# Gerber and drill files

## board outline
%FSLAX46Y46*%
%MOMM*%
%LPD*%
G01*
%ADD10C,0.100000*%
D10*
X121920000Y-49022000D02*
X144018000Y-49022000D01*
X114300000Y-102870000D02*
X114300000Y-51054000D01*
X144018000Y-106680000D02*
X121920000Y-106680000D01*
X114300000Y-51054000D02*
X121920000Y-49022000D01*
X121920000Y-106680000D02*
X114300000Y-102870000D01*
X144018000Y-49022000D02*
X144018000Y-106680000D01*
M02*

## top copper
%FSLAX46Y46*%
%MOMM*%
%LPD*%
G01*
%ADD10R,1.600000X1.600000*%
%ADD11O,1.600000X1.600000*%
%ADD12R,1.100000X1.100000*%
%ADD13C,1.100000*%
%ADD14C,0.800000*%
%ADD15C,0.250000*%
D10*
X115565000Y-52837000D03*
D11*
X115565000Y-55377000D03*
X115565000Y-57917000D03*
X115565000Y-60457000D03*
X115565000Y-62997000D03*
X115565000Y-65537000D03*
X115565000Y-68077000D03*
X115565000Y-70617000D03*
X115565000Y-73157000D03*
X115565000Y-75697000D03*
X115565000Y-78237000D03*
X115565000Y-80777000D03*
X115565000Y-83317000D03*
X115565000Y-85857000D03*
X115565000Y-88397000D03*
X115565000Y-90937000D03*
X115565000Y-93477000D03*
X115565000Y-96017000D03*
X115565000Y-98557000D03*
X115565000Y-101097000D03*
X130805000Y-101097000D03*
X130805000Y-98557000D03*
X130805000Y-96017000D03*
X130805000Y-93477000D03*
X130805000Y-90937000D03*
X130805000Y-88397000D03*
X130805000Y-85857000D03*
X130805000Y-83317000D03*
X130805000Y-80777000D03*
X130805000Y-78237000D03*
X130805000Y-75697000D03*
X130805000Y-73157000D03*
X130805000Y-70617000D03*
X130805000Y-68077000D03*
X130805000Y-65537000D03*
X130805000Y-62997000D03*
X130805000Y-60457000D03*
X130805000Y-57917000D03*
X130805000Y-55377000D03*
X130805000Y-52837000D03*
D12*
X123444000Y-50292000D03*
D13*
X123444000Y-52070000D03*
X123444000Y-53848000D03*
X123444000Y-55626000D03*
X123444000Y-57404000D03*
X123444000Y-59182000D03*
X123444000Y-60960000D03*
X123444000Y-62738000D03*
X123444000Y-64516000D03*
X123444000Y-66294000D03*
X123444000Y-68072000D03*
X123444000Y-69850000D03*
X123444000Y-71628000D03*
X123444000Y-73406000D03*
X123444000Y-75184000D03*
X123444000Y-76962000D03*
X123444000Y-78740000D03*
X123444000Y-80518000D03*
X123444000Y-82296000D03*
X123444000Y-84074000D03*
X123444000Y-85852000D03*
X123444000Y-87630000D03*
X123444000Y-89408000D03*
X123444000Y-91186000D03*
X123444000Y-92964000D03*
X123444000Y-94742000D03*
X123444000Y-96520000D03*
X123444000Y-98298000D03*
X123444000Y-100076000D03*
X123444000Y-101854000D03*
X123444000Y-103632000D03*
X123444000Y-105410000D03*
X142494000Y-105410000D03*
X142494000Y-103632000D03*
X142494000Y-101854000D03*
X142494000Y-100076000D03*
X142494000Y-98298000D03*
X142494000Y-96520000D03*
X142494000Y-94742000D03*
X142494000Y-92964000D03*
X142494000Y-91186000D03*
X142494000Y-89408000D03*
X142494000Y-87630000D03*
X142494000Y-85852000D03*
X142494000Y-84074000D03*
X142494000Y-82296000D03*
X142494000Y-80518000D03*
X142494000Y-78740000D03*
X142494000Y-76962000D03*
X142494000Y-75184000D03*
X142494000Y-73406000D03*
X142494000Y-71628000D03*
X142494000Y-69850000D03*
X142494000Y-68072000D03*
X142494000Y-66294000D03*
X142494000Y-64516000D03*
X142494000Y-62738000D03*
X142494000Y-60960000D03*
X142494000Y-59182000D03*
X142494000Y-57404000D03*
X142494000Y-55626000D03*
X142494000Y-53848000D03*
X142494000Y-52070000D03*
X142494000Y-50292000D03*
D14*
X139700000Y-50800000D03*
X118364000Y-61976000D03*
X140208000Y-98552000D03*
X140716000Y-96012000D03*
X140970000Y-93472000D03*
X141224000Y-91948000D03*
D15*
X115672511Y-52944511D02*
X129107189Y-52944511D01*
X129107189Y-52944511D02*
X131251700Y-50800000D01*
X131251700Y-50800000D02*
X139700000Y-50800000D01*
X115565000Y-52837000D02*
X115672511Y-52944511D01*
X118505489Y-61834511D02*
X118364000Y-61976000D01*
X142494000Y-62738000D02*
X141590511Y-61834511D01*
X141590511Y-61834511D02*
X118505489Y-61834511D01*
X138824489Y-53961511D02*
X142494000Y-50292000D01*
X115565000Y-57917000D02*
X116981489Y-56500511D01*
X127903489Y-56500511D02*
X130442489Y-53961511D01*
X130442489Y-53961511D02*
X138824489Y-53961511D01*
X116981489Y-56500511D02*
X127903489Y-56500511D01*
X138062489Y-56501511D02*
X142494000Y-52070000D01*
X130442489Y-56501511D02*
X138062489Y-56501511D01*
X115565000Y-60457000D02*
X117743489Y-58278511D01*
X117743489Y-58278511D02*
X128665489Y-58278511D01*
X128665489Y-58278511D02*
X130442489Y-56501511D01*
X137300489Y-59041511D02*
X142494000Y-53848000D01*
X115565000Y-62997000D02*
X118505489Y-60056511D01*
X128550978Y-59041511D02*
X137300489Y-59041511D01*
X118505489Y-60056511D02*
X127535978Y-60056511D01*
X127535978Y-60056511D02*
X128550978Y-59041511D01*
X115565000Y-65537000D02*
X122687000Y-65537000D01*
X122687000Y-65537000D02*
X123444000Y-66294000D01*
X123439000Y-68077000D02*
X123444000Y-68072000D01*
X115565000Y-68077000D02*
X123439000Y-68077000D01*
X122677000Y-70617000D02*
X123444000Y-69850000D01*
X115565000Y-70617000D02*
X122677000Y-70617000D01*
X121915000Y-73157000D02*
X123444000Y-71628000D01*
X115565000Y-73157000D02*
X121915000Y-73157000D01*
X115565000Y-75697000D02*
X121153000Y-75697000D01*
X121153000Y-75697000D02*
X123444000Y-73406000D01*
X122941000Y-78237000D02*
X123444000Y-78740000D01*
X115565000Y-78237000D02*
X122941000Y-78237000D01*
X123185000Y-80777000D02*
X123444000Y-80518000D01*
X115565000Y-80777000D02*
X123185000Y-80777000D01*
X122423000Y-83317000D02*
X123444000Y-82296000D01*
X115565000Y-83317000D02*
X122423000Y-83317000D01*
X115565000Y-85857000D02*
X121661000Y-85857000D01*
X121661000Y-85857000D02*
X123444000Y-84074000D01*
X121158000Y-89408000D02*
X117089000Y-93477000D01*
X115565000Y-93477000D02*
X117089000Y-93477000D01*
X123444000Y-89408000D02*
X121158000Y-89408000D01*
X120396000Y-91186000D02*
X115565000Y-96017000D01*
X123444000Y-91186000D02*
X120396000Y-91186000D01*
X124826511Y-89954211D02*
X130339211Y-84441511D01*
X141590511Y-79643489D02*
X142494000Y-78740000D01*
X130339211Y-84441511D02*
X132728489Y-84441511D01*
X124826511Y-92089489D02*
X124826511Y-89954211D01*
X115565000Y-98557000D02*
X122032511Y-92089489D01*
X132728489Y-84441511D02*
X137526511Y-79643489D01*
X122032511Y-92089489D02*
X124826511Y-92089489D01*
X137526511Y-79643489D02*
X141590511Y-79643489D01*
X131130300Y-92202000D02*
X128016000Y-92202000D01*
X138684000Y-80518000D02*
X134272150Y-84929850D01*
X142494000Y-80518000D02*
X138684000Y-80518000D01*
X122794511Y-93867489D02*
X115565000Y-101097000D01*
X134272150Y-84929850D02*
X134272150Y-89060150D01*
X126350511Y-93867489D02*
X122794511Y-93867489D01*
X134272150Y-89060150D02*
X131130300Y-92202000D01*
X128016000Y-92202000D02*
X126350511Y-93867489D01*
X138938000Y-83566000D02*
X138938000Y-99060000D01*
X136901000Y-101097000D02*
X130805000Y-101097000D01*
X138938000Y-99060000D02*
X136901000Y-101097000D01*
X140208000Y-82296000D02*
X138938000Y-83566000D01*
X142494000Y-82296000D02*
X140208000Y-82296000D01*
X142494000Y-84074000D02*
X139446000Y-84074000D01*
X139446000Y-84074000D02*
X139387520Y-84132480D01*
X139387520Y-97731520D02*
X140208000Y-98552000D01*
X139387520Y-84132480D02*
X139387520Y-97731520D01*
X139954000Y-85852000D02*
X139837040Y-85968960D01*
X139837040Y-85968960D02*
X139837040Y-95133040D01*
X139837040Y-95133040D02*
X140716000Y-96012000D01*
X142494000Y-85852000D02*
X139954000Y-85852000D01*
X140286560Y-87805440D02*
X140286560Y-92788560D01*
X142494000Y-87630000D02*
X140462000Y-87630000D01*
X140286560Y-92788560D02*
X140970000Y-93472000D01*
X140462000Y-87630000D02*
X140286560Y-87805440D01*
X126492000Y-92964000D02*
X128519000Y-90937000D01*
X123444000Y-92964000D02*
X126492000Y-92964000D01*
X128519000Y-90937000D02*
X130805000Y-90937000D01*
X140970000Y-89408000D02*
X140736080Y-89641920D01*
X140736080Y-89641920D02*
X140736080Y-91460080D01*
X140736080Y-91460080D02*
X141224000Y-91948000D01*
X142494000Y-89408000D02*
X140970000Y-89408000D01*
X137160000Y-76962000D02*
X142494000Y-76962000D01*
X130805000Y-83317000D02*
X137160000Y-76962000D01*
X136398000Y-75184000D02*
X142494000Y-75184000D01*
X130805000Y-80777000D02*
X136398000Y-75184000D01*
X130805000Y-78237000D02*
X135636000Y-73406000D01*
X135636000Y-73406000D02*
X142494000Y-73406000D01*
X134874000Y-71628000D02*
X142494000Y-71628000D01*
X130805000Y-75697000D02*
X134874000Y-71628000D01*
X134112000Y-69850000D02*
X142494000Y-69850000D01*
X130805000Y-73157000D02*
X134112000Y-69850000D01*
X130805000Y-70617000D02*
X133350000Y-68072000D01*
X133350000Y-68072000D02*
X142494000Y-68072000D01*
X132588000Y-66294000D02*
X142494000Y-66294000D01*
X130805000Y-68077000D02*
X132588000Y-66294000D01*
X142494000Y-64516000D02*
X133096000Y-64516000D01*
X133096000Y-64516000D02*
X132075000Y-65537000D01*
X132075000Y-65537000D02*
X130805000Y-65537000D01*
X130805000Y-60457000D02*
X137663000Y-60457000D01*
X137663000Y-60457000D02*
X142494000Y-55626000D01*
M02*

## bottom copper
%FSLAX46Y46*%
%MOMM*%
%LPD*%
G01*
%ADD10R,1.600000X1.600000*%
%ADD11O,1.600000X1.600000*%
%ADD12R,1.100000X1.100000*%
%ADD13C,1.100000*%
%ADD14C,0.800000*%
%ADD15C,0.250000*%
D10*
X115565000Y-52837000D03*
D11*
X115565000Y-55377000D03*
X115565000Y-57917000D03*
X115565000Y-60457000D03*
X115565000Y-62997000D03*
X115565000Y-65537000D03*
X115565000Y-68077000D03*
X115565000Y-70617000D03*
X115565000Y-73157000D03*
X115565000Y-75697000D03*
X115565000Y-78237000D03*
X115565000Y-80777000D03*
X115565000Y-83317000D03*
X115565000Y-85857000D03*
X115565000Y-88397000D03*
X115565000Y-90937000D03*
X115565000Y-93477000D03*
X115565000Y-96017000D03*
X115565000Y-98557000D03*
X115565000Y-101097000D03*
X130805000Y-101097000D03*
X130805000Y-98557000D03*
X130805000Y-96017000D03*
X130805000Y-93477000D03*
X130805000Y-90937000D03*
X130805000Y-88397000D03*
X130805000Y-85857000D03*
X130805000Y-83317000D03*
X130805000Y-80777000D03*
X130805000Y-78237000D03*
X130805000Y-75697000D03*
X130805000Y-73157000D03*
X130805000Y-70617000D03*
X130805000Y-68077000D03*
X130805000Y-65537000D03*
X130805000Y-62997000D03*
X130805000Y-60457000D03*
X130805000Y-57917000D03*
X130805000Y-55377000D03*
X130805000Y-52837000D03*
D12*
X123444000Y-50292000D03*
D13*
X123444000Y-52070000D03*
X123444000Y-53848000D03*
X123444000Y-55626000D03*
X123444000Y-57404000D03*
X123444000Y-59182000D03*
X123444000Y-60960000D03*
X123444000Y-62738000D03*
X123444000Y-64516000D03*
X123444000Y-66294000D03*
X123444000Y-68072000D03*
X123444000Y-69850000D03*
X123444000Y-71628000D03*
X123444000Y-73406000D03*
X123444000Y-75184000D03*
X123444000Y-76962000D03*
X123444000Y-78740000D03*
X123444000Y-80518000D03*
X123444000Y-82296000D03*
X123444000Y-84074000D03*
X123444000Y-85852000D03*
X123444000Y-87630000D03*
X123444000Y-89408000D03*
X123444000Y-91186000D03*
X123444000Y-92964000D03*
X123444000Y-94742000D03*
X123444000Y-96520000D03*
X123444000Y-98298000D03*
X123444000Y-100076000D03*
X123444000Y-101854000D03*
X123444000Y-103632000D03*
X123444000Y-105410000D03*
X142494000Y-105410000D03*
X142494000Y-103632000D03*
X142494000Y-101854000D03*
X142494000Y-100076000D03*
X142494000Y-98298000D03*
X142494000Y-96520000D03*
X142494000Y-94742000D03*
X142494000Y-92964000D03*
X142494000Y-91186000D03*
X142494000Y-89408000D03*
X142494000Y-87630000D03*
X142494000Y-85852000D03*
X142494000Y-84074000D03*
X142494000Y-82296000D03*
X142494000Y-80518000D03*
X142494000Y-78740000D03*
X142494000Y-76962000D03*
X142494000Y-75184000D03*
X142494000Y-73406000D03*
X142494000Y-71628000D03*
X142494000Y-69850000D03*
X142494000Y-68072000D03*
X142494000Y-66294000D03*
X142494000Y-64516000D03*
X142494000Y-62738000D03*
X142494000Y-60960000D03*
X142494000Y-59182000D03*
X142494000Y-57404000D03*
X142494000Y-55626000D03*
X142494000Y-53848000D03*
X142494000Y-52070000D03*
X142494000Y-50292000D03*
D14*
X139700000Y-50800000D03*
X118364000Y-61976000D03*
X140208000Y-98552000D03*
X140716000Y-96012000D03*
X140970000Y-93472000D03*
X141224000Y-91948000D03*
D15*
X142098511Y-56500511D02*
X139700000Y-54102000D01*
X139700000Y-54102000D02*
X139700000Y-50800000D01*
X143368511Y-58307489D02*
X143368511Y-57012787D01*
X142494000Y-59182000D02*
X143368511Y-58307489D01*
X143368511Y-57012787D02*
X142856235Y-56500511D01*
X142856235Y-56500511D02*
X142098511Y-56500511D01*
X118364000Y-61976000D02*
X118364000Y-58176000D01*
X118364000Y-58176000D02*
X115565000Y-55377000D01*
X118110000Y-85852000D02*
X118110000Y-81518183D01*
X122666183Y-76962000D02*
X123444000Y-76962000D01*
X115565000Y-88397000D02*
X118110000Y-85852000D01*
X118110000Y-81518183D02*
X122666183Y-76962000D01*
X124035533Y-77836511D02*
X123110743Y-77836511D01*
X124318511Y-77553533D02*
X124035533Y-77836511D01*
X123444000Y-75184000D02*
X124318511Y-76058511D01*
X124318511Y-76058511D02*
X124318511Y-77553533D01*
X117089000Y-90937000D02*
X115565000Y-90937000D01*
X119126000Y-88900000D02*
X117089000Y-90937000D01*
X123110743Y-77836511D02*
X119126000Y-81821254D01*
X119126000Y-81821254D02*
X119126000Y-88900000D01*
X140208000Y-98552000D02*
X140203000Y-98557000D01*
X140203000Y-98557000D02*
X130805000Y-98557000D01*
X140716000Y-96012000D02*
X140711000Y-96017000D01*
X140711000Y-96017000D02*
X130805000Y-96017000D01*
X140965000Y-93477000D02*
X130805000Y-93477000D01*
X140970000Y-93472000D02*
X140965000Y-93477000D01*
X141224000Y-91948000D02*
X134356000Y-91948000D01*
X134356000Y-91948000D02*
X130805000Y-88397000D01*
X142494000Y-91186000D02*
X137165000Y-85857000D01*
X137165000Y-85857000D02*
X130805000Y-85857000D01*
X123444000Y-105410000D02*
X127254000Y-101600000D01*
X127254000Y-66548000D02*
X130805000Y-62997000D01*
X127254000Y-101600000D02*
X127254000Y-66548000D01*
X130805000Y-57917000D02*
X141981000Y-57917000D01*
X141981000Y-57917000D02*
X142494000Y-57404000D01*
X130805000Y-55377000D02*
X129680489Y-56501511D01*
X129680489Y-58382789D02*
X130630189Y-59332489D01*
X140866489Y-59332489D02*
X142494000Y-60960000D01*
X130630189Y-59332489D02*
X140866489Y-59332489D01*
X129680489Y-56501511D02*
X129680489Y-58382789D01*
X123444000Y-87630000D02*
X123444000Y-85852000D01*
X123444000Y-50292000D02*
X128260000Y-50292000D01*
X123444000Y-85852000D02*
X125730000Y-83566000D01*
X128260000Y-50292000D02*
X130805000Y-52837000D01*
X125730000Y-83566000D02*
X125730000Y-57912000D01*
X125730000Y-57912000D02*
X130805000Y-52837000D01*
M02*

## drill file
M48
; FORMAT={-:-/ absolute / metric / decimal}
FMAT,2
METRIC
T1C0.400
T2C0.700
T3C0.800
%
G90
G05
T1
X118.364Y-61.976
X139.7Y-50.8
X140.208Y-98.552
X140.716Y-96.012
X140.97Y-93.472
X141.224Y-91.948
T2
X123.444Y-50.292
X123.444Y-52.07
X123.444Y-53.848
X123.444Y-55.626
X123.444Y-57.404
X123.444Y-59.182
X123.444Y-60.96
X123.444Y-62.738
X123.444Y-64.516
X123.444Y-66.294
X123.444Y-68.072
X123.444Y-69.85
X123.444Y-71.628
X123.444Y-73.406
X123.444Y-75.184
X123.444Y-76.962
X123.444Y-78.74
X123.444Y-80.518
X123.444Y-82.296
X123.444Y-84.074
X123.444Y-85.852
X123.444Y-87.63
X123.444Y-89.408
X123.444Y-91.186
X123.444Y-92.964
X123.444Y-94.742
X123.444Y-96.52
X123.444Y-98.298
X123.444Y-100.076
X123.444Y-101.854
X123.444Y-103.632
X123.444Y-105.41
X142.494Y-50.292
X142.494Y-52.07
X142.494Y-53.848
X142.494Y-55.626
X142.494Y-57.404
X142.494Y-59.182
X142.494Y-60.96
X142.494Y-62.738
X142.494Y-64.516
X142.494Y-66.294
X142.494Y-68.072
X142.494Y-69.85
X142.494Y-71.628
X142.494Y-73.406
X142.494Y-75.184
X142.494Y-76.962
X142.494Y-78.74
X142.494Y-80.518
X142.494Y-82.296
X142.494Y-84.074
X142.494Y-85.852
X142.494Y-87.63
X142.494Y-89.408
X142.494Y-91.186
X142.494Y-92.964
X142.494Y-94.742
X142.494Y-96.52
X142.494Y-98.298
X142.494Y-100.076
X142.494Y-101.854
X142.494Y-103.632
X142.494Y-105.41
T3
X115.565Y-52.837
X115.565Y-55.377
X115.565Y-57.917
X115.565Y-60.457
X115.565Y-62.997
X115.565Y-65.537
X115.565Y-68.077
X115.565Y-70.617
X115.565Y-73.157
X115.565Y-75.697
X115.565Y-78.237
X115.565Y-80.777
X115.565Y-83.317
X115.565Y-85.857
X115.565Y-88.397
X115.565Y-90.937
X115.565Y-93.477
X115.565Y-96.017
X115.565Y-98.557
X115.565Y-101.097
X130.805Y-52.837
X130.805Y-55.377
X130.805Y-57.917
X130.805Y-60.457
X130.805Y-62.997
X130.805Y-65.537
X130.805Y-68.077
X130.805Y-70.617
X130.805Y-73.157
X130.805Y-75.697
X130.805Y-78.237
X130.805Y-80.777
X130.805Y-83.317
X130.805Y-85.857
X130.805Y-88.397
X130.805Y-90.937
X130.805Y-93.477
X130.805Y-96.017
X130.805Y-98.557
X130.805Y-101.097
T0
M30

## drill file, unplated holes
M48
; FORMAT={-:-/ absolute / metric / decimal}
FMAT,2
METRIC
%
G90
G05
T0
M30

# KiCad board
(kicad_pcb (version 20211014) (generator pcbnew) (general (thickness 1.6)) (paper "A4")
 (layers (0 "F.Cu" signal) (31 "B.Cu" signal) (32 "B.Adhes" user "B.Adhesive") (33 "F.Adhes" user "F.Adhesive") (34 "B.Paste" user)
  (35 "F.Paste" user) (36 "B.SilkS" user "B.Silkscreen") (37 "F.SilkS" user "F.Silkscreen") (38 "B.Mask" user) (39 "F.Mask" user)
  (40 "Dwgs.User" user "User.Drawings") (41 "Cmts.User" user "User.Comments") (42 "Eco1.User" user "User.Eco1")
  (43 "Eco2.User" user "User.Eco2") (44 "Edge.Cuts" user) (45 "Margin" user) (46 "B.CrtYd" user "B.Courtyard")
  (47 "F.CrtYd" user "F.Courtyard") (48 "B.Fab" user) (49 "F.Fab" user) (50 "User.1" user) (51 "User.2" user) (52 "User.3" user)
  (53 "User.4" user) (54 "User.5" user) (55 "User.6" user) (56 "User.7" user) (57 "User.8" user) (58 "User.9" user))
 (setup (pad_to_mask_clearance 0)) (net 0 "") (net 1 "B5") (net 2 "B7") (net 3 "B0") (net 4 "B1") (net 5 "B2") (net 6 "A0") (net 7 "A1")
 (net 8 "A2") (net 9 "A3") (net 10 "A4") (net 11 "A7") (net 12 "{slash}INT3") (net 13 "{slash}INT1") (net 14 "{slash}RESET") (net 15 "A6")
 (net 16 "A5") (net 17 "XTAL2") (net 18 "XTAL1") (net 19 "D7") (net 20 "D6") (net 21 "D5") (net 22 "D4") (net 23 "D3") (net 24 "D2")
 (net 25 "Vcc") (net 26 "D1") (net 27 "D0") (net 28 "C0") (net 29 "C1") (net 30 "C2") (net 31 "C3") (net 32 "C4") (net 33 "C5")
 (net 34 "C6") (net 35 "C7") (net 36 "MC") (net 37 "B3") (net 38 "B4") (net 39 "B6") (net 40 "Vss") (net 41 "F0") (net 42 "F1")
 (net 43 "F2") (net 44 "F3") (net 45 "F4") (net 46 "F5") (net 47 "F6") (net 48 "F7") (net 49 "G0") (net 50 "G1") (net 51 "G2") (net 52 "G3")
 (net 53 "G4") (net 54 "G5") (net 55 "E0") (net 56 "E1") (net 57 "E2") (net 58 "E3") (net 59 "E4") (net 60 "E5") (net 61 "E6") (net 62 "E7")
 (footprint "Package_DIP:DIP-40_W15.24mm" (layer "F.Cu") (at 115.565 52.837)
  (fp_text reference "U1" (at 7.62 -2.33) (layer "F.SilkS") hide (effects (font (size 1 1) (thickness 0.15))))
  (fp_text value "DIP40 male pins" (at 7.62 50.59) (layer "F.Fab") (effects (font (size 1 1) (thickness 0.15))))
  (pad "1" thru_hole rect locked (at 0 0) (size 1.6 1.6) (drill 0.8) (layers *.Cu *.Mask) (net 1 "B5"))
  (pad "2" thru_hole oval locked (at 0 2.54) (size 1.6 1.6) (drill 0.8) (layers *.Cu *.Mask) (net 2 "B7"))
  (pad "3" thru_hole oval locked (at 0 5.08) (size 1.6 1.6) (drill 0.8) (layers *.Cu *.Mask) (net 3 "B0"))
  (pad "4" thru_hole oval locked (at 0 7.62) (size 1.6 1.6) (drill 0.8) (layers *.Cu *.Mask) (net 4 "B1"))
  (pad "5" thru_hole oval locked (at 0 10.16) (size 1.6 1.6) (drill 0.8) (layers *.Cu *.Mask) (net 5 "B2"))
  (pad "6" thru_hole oval locked (at 0 12.7) (size 1.6 1.6) (drill 0.8) (layers *.Cu *.Mask) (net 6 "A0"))
  (pad "7" thru_hole oval locked (at 0 15.24) (size 1.6 1.6) (drill 0.8) (layers *.Cu *.Mask) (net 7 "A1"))
  (pad "8" thru_hole oval locked (at 0 17.78) (size 1.6 1.6) (drill 0.8) (layers *.Cu *.Mask) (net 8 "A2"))
  (pad "9" thru_hole oval locked (at 0 20.32) (size 1.6 1.6) (drill 0.8) (layers *.Cu *.Mask) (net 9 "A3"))
  (pad "10" thru_hole oval locked (at 0 22.86) (size 1.6 1.6) (drill 0.8) (layers *.Cu *.Mask) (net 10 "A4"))
  (pad "11" thru_hole oval locked (at 0 25.4) (size 1.6 1.6) (drill 0.8) (layers *.Cu *.Mask) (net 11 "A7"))
  (pad "12" thru_hole oval locked (at 0 27.94) (size 1.6 1.6) (drill 0.8) (layers *.Cu *.Mask) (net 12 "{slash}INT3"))
  (pad "13" thru_hole oval locked (at 0 30.48) (size 1.6 1.6) (drill 0.8) (layers *.Cu *.Mask) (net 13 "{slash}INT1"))
  (pad "14" thru_hole oval locked (at 0 33.02) (size 1.6 1.6) (drill 0.8) (layers *.Cu *.Mask) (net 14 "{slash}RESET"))
  (pad "15" thru_hole oval locked (at 0 35.56) (size 1.6 1.6) (drill 0.8) (layers *.Cu *.Mask) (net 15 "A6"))
  (pad "16" thru_hole oval locked (at 0 38.1) (size 1.6 1.6) (drill 0.8) (layers *.Cu *.Mask) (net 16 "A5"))
  (pad "17" thru_hole oval locked (at 0 40.64) (size 1.6 1.6) (drill 0.8) (layers *.Cu *.Mask) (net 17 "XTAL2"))
  (pad "18" thru_hole oval locked (at 0 43.18) (size 1.6 1.6) (drill 0.8) (layers *.Cu *.Mask) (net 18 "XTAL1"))
  (pad "19" thru_hole oval locked (at 0 45.72) (size 1.6 1.6) (drill 0.8) (layers *.Cu *.Mask) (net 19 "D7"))
  (pad "20" thru_hole oval locked (at 0 48.26) (size 1.6 1.6) (drill 0.8) (layers *.Cu *.Mask) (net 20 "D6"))
  (pad "21" thru_hole oval locked (at 15.24 48.26) (size 1.6 1.6) (drill 0.8) (layers *.Cu *.Mask) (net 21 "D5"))
  (pad "22" thru_hole oval locked (at 15.24 45.72) (size 1.6 1.6) (drill 0.8) (layers *.Cu *.Mask) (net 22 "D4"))
  (pad "23" thru_hole oval locked (at 15.24 43.18) (size 1.6 1.6) (drill 0.8) (layers *.Cu *.Mask) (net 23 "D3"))
  (pad "24" thru_hole oval locked (at 15.24 40.64) (size 1.6 1.6) (drill 0.8) (layers *.Cu *.Mask) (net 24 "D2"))
  (pad "25" thru_hole oval locked (at 15.24 38.1) (size 1.6 1.6) (drill 0.8) (layers *.Cu *.Mask) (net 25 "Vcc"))
  (pad "26" thru_hole oval locked (at 15.24 35.56) (size 1.6 1.6) (drill 0.8) (layers *.Cu *.Mask) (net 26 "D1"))
  (pad "27" thru_hole oval locked (at 15.24 33.02) (size 1.6 1.6) (drill 0.8) (layers *.Cu *.Mask) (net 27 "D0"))
  (pad "28" thru_hole oval locked (at 15.24 30.48) (size 1.6 1.6) (drill 0.8) (layers *.Cu *.Mask) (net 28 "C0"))
  (pad "29" thru_hole oval locked (at 15.24 27.94) (size 1.6 1.6) (drill 0.8) (layers *.Cu *.Mask) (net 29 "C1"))
  (pad "30" thru_hole oval locked (at 15.24 25.4) (size 1.6 1.6) (drill 0.8) (layers *.Cu *.Mask) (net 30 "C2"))
  (pad "31" thru_hole oval locked (at 15.24 22.86) (size 1.6 1.6) (drill 0.8) (layers *.Cu *.Mask) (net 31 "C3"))
  (pad "32" thru_hole oval locked (at 15.24 20.32) (size 1.6 1.6) (drill 0.8) (layers *.Cu *.Mask) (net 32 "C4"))
  (pad "33" thru_hole oval locked (at 15.24 17.78) (size 1.6 1.6) (drill 0.8) (layers *.Cu *.Mask) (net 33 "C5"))
  (pad "34" thru_hole oval locked (at 15.24 15.24) (size 1.6 1.6) (drill 0.8) (layers *.Cu *.Mask) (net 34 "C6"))
  (pad "35" thru_hole oval locked (at 15.24 12.7) (size 1.6 1.6) (drill 0.8) (layers *.Cu *.Mask) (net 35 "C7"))
  (pad "36" thru_hole oval locked (at 15.24 10.16) (size 1.6 1.6) (drill 0.8) (layers *.Cu *.Mask) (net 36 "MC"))
  (pad "37" thru_hole oval locked (at 15.24 7.62) (size 1.6 1.6) (drill 0.8) (layers *.Cu *.Mask) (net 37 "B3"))
  (pad "38" thru_hole oval locked (at 15.24 5.08) (size 1.6 1.6) (drill 0.8) (layers *.Cu *.Mask) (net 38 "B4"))
  (pad "39" thru_hole oval locked (at 15.24 2.54) (size 1.6 1.6) (drill 0.8) (layers *.Cu *.Mask) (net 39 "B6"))
  (pad "40" thru_hole oval locked (at 15.24 0) (size 1.6 1.6) (drill 0.8) (layers *.Cu *.Mask) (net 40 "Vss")))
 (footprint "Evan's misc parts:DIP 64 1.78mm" (layer "F.Cu") (at 123.444 50.292)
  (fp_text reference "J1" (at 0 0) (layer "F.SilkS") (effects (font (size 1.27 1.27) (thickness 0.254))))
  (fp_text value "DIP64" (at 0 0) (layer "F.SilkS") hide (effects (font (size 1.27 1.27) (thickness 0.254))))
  (pad "1" thru_hole rect (at 0 0) (size 1.1 1.1) (drill 0.7) (layers *.Cu *.Mask) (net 40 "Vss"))
  (pad "2" thru_hole circle (at 0 1.778) (size 1.1 1.1) (drill 0.7) (layers *.Cu *.Mask) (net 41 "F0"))
  (pad "3" thru_hole circle (at 0 3.556) (size 1.1 1.1) (drill 0.7) (layers *.Cu *.Mask) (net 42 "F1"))
  (pad "4" thru_hole circle (at 0 5.334) (size 1.1 1.1) (drill 0.7) (layers *.Cu *.Mask) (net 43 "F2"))
  (pad "5" thru_hole circle (at 0 7.112) (size 1.1 1.1) (drill 0.7) (layers *.Cu *.Mask) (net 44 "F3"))
  (pad "6" thru_hole circle (at 0 8.89) (size 1.1 1.1) (drill 0.7) (layers *.Cu *.Mask) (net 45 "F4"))
  (pad "7" thru_hole circle (at 0 10.668) (size 1.1 1.1) (drill 0.7) (layers *.Cu *.Mask) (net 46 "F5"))
  (pad "8" thru_hole circle (at 0 12.446) (size 1.1 1.1) (drill 0.7) (layers *.Cu *.Mask) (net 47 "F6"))
  (pad "9" thru_hole circle (at 0 14.224) (size 1.1 1.1) (drill 0.7) (layers *.Cu *.Mask) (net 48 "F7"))
  (pad "10" thru_hole circle (at 0 16.002) (size 1.1 1.1) (drill 0.7) (layers *.Cu *.Mask) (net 6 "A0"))
  (pad "11" thru_hole circle (at 0 17.78) (size 1.1 1.1) (drill 0.7) (layers *.Cu *.Mask) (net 7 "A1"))
  (pad "12" thru_hole circle (at 0 19.558) (size 1.1 1.1) (drill 0.7) (layers *.Cu *.Mask) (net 8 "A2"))
  (pad "13" thru_hole circle (at 0 21.336) (size 1.1 1.1) (drill 0.7) (layers *.Cu *.Mask) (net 9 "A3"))
  (pad "14" thru_hole circle (at 0 23.114) (size 1.1 1.1) (drill 0.7) (layers *.Cu *.Mask) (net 10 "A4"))
  (pad "15" thru_hole circle (at 0 24.892) (size 1.1 1.1) (drill 0.7) (layers *.Cu *.Mask) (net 16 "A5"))
  (pad "16" thru_hole circle (at 0 26.67) (size 1.1 1.1) (drill 0.7) (layers *.Cu *.Mask) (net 15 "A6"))
  (pad "17" thru_hole circle (at 0 28.448) (size 1.1 1.1) (drill 0.7) (layers *.Cu *.Mask) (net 11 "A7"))
  (pad "18" thru_hole circle (at 0 30.226) (size 1.1 1.1) (drill 0.7) (layers *.Cu *.Mask) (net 12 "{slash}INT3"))
  (pad "19" thru_hole circle (at 0 32.004) (size 1.1 1.1) (drill 0.7) (layers *.Cu *.Mask) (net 13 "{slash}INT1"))
  (pad "20" thru_hole circle (at 0 33.782) (size 1.1 1.1) (drill 0.7) (layers *.Cu *.Mask) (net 14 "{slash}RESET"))
  (pad "21" thru_hole circle (at 0 35.56) (size 1.1 1.1) (drill 0.7) (layers *.Cu *.Mask) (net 40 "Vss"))
  (pad "22" thru_hole circle (at 0 37.338) (size 1.1 1.1) (drill 0.7) (layers *.Cu *.Mask) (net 40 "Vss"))
  (pad "23" thru_hole circle (at 0 39.116) (size 1.1 1.1) (drill 0.7) (layers *.Cu *.Mask) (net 17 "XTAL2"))
  (pad "24" thru_hole circle (at 0 40.894) (size 1.1 1.1) (drill 0.7) (layers *.Cu *.Mask) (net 18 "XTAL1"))
  (pad "25" thru_hole circle (at 0 42.672) (size 1.1 1.1) (drill 0.7) (layers *.Cu *.Mask) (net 25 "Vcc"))
  (pad "26" thru_hole circle (at 0 44.45) (size 1.1 1.1) (drill 0.7) (layers *.Cu *.Mask) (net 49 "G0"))
  (pad "27" thru_hole circle (at 0 46.228) (size 1.1 1.1) (drill 0.7) (layers *.Cu *.Mask) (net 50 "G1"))
  (pad "28" thru_hole circle (at 0 48.006) (size 1.1 1.1) (drill 0.7) (layers *.Cu *.Mask) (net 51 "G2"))
  (pad "29" thru_hole circle (at 0 49.784) (size 1.1 1.1) (drill 0.7) (layers *.Cu *.Mask) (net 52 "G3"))
  (pad "30" thru_hole circle (at 0 51.562) (size 1.1 1.1) (drill 0.7) (layers *.Cu *.Mask) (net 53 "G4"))
  (pad "31" thru_hole circle (at 0 53.34) (size 1.1 1.1) (drill 0.7) (layers *.Cu *.Mask) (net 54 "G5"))
  (pad "32" thru_hole circle (at 0 55.118) (size 1.1 1.1) (drill 0.7) (layers *.Cu *.Mask) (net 36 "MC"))
  (pad "33" thru_hole circle (at 19.05 55.118) (size 1.1 1.1) (drill 0.7) (layers *.Cu *.Mask) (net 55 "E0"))
  (pad "34" thru_hole circle (at 19.05 53.34) (size 1.1 1.1) (drill 0.7) (layers *.Cu *.Mask) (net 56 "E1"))
  (pad "35" thru_hole circle (at 19.05 51.562) (size 1.1 1.1) (drill 0.7) (layers *.Cu *.Mask) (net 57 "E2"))
  (pad "36" thru_hole circle (at 19.05 49.784) (size 1.1 1.1) (drill 0.7) (layers *.Cu *.Mask) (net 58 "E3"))
  (pad "37" thru_hole circle (at 19.05 48.006) (size 1.1 1.1) (drill 0.7) (layers *.Cu *.Mask) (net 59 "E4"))
  (pad "38" thru_hole circle (at 19.05 46.228) (size 1.1 1.1) (drill 0.7) (layers *.Cu *.Mask) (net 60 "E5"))
  (pad "39" thru_hole circle (at 19.05 44.45) (size 1.1 1.1) (drill 0.7) (layers *.Cu *.Mask) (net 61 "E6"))
  (pad "40" thru_hole circle (at 19.05 42.672) (size 1.1 1.1) (drill 0.7) (layers *.Cu *.Mask) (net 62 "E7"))
  (pad "41" thru_hole circle (at 19.05 40.894) (size 1.1 1.1) (drill 0.7) (layers *.Cu *.Mask) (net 27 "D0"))
  (pad "42" thru_hole circle (at 19.05 39.116) (size 1.1 1.1) (drill 0.7) (layers *.Cu *.Mask) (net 26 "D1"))
  (pad "43" thru_hole circle (at 19.05 37.338) (size 1.1 1.1) (drill 0.7) (layers *.Cu *.Mask) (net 24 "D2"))
  (pad "44" thru_hole circle (at 19.05 35.56) (size 1.1 1.1) (drill 0.7) (layers *.Cu *.Mask) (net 23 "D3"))
  (pad "45" thru_hole circle (at 19.05 33.782) (size 1.1 1.1) (drill 0.7) (layers *.Cu *.Mask) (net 22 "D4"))
  (pad "46" thru_hole circle (at 19.05 32.004) (size 1.1 1.1) (drill 0.7) (layers *.Cu *.Mask) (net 21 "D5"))
  (pad "47" thru_hole circle (at 19.05 30.226) (size 1.1 1.1) (drill 0.7) (layers *.Cu *.Mask) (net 20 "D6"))
  (pad "48" thru_hole circle (at 19.05 28.448) (size 1.1 1.1) (drill 0.7) (layers *.Cu *.Mask) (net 19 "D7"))
  (pad "49" thru_hole circle (at 19.05 26.67) (size 1.1 1.1) (drill 0.7) (layers *.Cu *.Mask) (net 28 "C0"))
  (pad "50" thru_hole circle (at 19.05 24.892) (size 1.1 1.1) (drill 0.7) (layers *.Cu *.Mask) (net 29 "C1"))
  (pad "51" thru_hole circle (at 19.05 23.114) (size 1.1 1.1) (drill 0.7) (layers *.Cu *.Mask) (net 30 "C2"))
  (pad "52" thru_hole circle (at 19.05 21.336) (size 1.1 1.1) (drill 0.7) (layers *.Cu *.Mask) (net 31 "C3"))
  (pad "53" thru_hole circle (at 19.05 19.558) (size 1.1 1.1) (drill 0.7) (layers *.Cu *.Mask) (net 32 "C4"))
  (pad "54" thru_hole circle (at 19.05 17.78) (size 1.1 1.1) (drill 0.7) (layers *.Cu *.Mask) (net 33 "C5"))
  (pad "55" thru_hole circle (at 19.05 16.002) (size 1.1 1.1) (drill 0.7) (layers *.Cu *.Mask) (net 34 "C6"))
  (pad "56" thru_hole circle (at 19.05 14.224) (size 1.1 1.1) (drill 0.7) (layers *.Cu *.Mask) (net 35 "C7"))
  (pad "57" thru_hole circle (at 19.05 12.446) (size 1.1 1.1) (drill 0.7) (layers *.Cu *.Mask) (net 2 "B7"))
  (pad "58" thru_hole circle (at 19.05 10.668) (size 1.1 1.1) (drill 0.7) (layers *.Cu *.Mask) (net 39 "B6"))
  (pad "59" thru_hole circle (at 19.05 8.89) (size 1.1 1.1) (drill 0.7) (layers *.Cu *.Mask) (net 1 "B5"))
  (pad "60" thru_hole circle (at 19.05 7.112) (size 1.1 1.1) (drill 0.7) (layers *.Cu *.Mask) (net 38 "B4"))
  (pad "61" thru_hole circle (at 19.05 5.334) (size 1.1 1.1) (drill 0.7) (layers *.Cu *.Mask) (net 37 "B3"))
  (pad "62" thru_hole circle (at 19.05 3.556) (size 1.1 1.1) (drill 0.7) (layers *.Cu *.Mask) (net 5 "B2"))
  (pad "63" thru_hole circle (at 19.05 1.778) (size 1.1 1.1) (drill 0.7) (layers *.Cu *.Mask) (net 4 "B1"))
  (pad "64" thru_hole circle (at 19.05 0) (size 1.1 1.1) (drill 0.7) (layers *.Cu *.Mask) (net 3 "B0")))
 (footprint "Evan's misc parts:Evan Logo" (layer "F.Cu") (at 119.38 98.298 90)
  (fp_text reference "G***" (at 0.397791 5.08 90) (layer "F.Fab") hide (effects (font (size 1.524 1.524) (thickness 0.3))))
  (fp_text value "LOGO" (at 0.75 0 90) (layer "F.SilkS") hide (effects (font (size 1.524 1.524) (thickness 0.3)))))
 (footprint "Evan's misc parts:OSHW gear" (layer "B.Cu") (at 135.382 100.838 -90)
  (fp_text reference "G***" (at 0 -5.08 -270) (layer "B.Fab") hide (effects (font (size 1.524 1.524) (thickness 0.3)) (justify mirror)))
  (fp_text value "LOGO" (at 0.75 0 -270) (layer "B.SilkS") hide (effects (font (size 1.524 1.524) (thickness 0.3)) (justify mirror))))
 (gr_line (start 121.92 49.022) (end 144.018 49.022) (layer "Edge.Cuts") (width 0.1))
 (gr_line (start 114.3 102.87) (end 114.3 51.054) (layer "Edge.Cuts") (width 0.1))
 (gr_line (start 144.018 106.68) (end 121.92 106.68) (layer "Edge.Cuts") (width 0.1))
 (gr_line (start 114.3 51.054) (end 121.92 49.022) (layer "Edge.Cuts") (width 0.1))
 (gr_line (start 121.92 106.68) (end 114.3 102.87) (layer "Edge.Cuts") (width 0.1))
 (gr_line (start 144.018 49.022) (end 144.018 106.68) (layer "Edge.Cuts") (width 0.1))
 (segment (start 115.672511 52.944511) (end 129.107189 52.944511) (width 0.25) (layer "F.Cu") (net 1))
 (segment (start 129.107189 52.944511) (end 131.2517 50.8) (width 0.25) (layer "F.Cu") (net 1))
 (segment (start 131.2517 50.8) (end 139.7 50.8) (width 0.25) (layer "F.Cu") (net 1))
 (segment (start 115.565 52.837) (end 115.672511 52.944511) (width 0.25) (layer "F.Cu") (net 1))
 (via (at 139.7 50.8) (size 0.8) (drill 0.4) (layers "F.Cu" "B.Cu") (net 1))
 (segment (start 142.098511 56.500511) (end 139.7 54.102) (width 0.25) (layer "B.Cu") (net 1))
 (segment (start 139.7 54.102) (end 139.7 50.8) (width 0.25) (layer "B.Cu") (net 1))
 (segment (start 143.368511 58.307489) (end 143.368511 57.012787) (width 0.25) (layer "B.Cu") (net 1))
 (segment (start 142.494 59.182) (end 143.368511 58.307489) (width 0.25) (layer "B.Cu") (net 1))
 (segment (start 143.368511 57.012787) (end 142.856235 56.500511) (width 0.25) (layer "B.Cu") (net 1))
 (segment (start 142.856235 56.500511) (end 142.098511 56.500511) (width 0.25) (layer "B.Cu") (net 1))
 (segment (start 118.505489 61.834511) (end 118.364 61.976) (width 0.25) (layer "F.Cu") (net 2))
 (segment (start 142.494 62.738) (end 141.590511 61.834511) (width 0.25) (layer "F.Cu") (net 2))
 (segment (start 141.590511 61.834511) (end 118.505489 61.834511) (width 0.25) (layer "F.Cu") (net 2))
 (via (at 118.364 61.976) (size 0.8) (drill 0.4) (layers "F.Cu" "B.Cu") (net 2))
 (segment (start 118.364 61.976) (end 118.364 58.176) (width 0.25) (layer "B.Cu") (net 2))
 (segment (start 118.364 58.176) (end 115.565 55.377) (width 0.25) (layer "B.Cu") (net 2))
 (segment (start 138.824489 53.961511) (end 142.494 50.292) (width 0.25) (layer "F.Cu") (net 3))
 (segment (start 115.565 57.917) (end 116.981489 56.500511) (width 0.25) (layer "F.Cu") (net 3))
 (segment (start 127.903489 56.500511) (end 130.442489 53.961511) (width 0.25) (layer "F.Cu") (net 3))
 (segment (start 130.442489 53.961511) (end 138.824489 53.961511) (width 0.25) (layer "F.Cu") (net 3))
 (segment (start 116.981489 56.500511) (end 127.903489 56.500511) (width 0.25) (layer "F.Cu") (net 3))
 (segment (start 138.062489 56.501511) (end 142.494 52.07) (width 0.25) (layer "F.Cu") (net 4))
 (segment (start 130.442489 56.501511) (end 138.062489 56.501511) (width 0.25) (layer "F.Cu") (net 4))
 (segment (start 115.565 60.457) (end 117.743489 58.278511) (width 0.25) (layer "F.Cu") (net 4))
 (segment (start 117.743489 58.278511) (end 128.665489 58.278511) (width 0.25) (layer "F.Cu") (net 4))
 (segment (start 128.665489 58.278511) (end 130.442489 56.501511) (width 0.25) (layer "F.Cu") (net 4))
 (segment (start 137.300489 59.041511) (end 142.494 53.848) (width 0.25) (layer "F.Cu") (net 5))
 (segment (start 115.565 62.997) (end 118.505489 60.056511) (width 0.25) (layer "F.Cu") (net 5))
 (segment (start 128.550978 59.041511) (end 137.300489 59.041511) (width 0.25) (layer "F.Cu") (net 5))
 (segment (start 118.505489 60.056511) (end 127.535978 60.056511) (width 0.25) (layer "F.Cu") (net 5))
 (segment (start 127.535978 60.056511) (end 128.550978 59.041511) (width 0.25) (layer "F.Cu") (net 5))
 (segment (start 115.565 65.537) (end 122.687 65.537) (width 0.25) (layer "F.Cu") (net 6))
 (segment (start 122.687 65.537) (end 123.444 66.294) (width 0.25) (layer "F.Cu") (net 6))
 (segment (start 123.439 68.077) (end 123.444 68.072) (width 0.25) (layer "F.Cu") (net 7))
 (segment (start 115.565 68.077) (end 123.439 68.077) (width 0.25) (layer "F.Cu") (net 7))
 (segment (start 122.677 70.617) (end 123.444 69.85) (width 0.25) (layer "F.Cu") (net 8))
 (segment (start 115.565 70.617) (end 122.677 70.617) (width 0.25) (layer "F.Cu") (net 8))
 (segment (start 121.915 73.157) (end 123.444 71.628) (width 0.25) (layer "F.Cu") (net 9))
 (segment (start 115.565 73.157) (end 121.915 73.157) (width 0.25) (layer "F.Cu") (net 9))
 (segment (start 115.565 75.697) (end 121.153 75.697) (width 0.25) (layer "F.Cu") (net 10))
 (segment (start 121.153 75.697) (end 123.444 73.406) (width 0.25) (layer "F.Cu") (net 10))
 (segment (start 122.941 78.237) (end 123.444 78.74) (width 0.25) (layer "F.Cu") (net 11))
 (segment (start 115.565 78.237) (end 122.941 78.237) (width 0.25) (layer "F.Cu") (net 11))
 (segment (start 123.185 80.777) (end 123.444 80.518) (width 0.25) (layer "F.Cu") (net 12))
 (segment (start 115.565 80.777) (end 123.185 80.777) (width 0.25) (layer "F.Cu") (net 12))
 (segment (start 122.423 83.317) (end 123.444 82.296) (width 0.25) (layer "F.Cu") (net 13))
 (segment (start 115.565 83.317) (end 122.423 83.317) (width 0.25) (layer "F.Cu") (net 13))
 (segment (start 115.565 85.857) (end 121.661 85.857) (width 0.25) (layer "F.Cu") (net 14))
 (segment (start 121.661 85.857) (end 123.444 84.074) (width 0.25) (layer "F.Cu") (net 14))
 (segment (start 118.11 85.852) (end 118.11 81.518183) (width 0.25) (layer "B.Cu") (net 15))
 (segment (start 122.666183 76.962) (end 123.444 76.962) (width 0.25) (layer "B.Cu") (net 15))
 (segment (start 115.565 88.397) (end 118.11 85.852) (width 0.25) (layer "B.Cu") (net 15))
 (segment (start 118.11 81.518183) (end 122.666183 76.962) (width 0.25) (layer "B.Cu") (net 15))
 (segment (start 124.035533 77.836511) (end 123.110743 77.836511) (width 0.25) (layer "B.Cu") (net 16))
 (segment (start 124.318511 77.553533) (end 124.035533 77.836511) (width 0.25) (layer "B.Cu") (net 16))
 (segment (start 123.444 75.184) (end 124.318511 76.058511) (width 0.25) (layer "B.Cu") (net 16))
 (segment (start 124.318511 76.058511) (end 124.318511 77.553533) (width 0.25) (layer "B.Cu") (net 16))
 (segment (start 117.089 90.937) (end 115.565 90.937) (width 0.25) (layer "B.Cu") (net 16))
 (segment (start 119.126 88.9) (end 117.089 90.937) (width 0.25) (layer "B.Cu") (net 16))
 (segment (start 123.110743 77.836511) (end 119.126 81.821254) (width 0.25) (layer "B.Cu") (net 16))
 (segment (start 119.126 81.821254) (end 119.126 88.9) (width 0.25) (layer "B.Cu") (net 16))
 (segment (start 121.158 89.408) (end 117.089 93.477) (width 0.25) (layer "F.Cu") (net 17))
 (segment (start 115.565 93.477) (end 117.089 93.477) (width 0.25) (layer "F.Cu") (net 17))
 (segment (start 123.444 89.408) (end 121.158 89.408) (width 0.25) (layer "F.Cu") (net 17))
 (segment (start 120.396 91.186) (end 115.565 96.017) (width 0.25) (layer "F.Cu") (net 18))
 (segment (start 123.444 91.186) (end 120.396 91.186) (width 0.25) (layer "F.Cu") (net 18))
 (segment (start 124.826511 89.954211) (end 130.339211 84.441511) (width 0.25) (layer "F.Cu") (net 19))
 (segment (start 141.590511 79.643489) (end 142.494 78.74) (width 0.25) (layer "F.Cu") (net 19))
 (segment (start 130.339211 84.441511) (end 132.728489 84.441511) (width 0.25) (layer "F.Cu") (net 19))
 (segment (start 124.826511 92.089489) (end 124.826511 89.954211) (width 0.25) (layer "F.Cu") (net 19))
 (segment (start 115.565 98.557) (end 122.032511 92.089489) (width 0.25) (layer "F.Cu") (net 19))
 (segment (start 132.728489 84.441511) (end 137.526511 79.643489) (width 0.25) (layer "F.Cu") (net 19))
 (segment (start 122.032511 92.089489) (end 124.826511 92.089489) (width 0.25) (layer "F.Cu") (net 19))
 (segment (start 137.526511 79.643489) (end 141.590511 79.643489) (width 0.25) (layer "F.Cu") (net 19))
 (segment (start 131.1303 92.202) (end 128.016 92.202) (width 0.25) (layer "F.Cu") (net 20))
 (segment (start 138.684 80.518) (end 134.27215 84.92985) (width 0.25) (layer "F.Cu") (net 20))
 (segment (start 142.494 80.518) (end 138.684 80.518) (width 0.25) (layer "F.Cu") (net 20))
 (segment (start 122.794511 93.867489) (end 115.565 101.097) (width 0.25) (layer "F.Cu") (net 20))
 (segment (start 134.27215 84.92985) (end 134.27215 89.06015) (width 0.25) (layer "F.Cu") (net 20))
 (segment (start 126.350511 93.867489) (end 122.794511 93.867489) (width 0.25) (layer "F.Cu") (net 20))
 (segment (start 134.27215 89.06015) (end 131.1303 92.202) (width 0.25) (layer "F.Cu") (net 20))
 (segment (start 128.016 92.202) (end 126.350511 93.867489) (width 0.25) (layer "F.Cu") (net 20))
 (segment (start 138.938 83.566) (end 138.938 99.06) (width 0.25) (layer "F.Cu") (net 21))
 (segment (start 136.901 101.097) (end 130.805 101.097) (width 0.25) (layer "F.Cu") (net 21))
 (segment (start 138.938 99.06) (end 136.901 101.097) (width 0.25) (layer "F.Cu") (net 21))
 (segment (start 140.208 82.296) (end 138.938 83.566) (width 0.25) (layer "F.Cu") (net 21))
 (segment (start 142.494 82.296) (end 140.208 82.296) (width 0.25) (layer "F.Cu") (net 21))
 (segment (start 142.494 84.074) (end 139.446 84.074) (width 0.25) (layer "F.Cu") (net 22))
 (segment (start 139.446 84.074) (end 139.38752 84.13248) (width 0.25) (layer "F.Cu") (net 22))
 (segment (start 139.38752 97.73152) (end 140.208 98.552) (width 0.25) (layer "F.Cu") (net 22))
 (segment (start 139.38752 84.13248) (end 139.38752 97.73152) (width 0.25) (layer "F.Cu") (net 22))
 (via (at 140.208 98.552) (size 0.8) (drill 0.4) (layers "F.Cu" "B.Cu") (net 22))
 (segment (start 140.208 98.552) (end 140.203 98.557) (width 0.25) (layer "B.Cu") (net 22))
 (segment (start 140.203 98.557) (end 130.805 98.557) (width 0.25) (layer "B.Cu") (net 22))
 (segment (start 139.954 85.852) (end 139.83704 85.96896) (width 0.25) (layer "F.Cu") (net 23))
 (segment (start 139.83704 85.96896) (end 139.83704 95.13304) (width 0.25) (layer "F.Cu") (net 23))
 (segment (start 139.83704 95.13304) (end 140.716 96.012) (width 0.25) (layer "F.Cu") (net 23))
 (segment (start 142.494 85.852) (end 139.954 85.852) (width 0.25) (layer "F.Cu") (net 23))
 (via (at 140.716 96.012) (size 0.8) (drill 0.4) (layers "F.Cu" "B.Cu") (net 23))
 (segment (start 140.716 96.012) (end 140.711 96.017) (width 0.25) (layer "B.Cu") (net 23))
 (segment (start 140.711 96.017) (end 130.805 96.017) (width 0.25) (layer "B.Cu") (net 23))
 (segment (start 140.28656 87.80544) (end 140.28656 92.78856) (width 0.25) (layer "F.Cu") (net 24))
 (segment (start 142.494 87.63) (end 140.462 87.63) (width 0.25) (layer "F.Cu") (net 24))
 (segment (start 140.28656 92.78856) (end 140.97 93.472) (width 0.25) (layer "F.Cu") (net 24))
 (segment (start 140.462 87.63) (end 140.28656 87.80544) (width 0.25) (layer "F.Cu") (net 24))
 (via (at 140.97 93.472) (size 0.8) (drill 0.4) (layers "F.Cu" "B.Cu") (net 24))
 (segment (start 140.965 93.477) (end 130.805 93.477) (width 0.25) (layer "B.Cu") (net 24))
 (segment (start 140.97 93.472) (end 140.965 93.477) (width 0.25) (layer "B.Cu") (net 24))
 (segment (start 126.492 92.964) (end 128.519 90.937) (width 0.25) (layer "F.Cu") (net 25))
 (segment (start 123.444 92.964) (end 126.492 92.964) (width 0.25) (layer "F.Cu") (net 25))
 (segment (start 128.519 90.937) (end 130.805 90.937) (width 0.25) (layer "F.Cu") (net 25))
 (segment (start 140.97 89.408) (end 140.73608 89.64192) (width 0.25) (layer "F.Cu") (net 26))
 (segment (start 140.73608 89.64192) (end 140.73608 91.46008) (width 0.25) (layer "F.Cu") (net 26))
 (segment (start 140.73608 91.46008) (end 141.224 91.948) (width 0.25) (layer "F.Cu") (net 26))
 (segment (start 142.494 89.408) (end 140.97 89.408) (width 0.25) (layer "F.Cu") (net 26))
 (via (at 141.224 91.948) (size 0.8) (drill 0.4) (layers "F.Cu" "B.Cu") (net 26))
 (segment (start 141.224 91.948) (end 134.356 91.948) (width 0.25) (layer "B.Cu") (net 26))
 (segment (start 134.356 91.948) (end 130.805 88.397) (width 0.25) (layer "B.Cu") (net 26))
 (segment (start 142.494 91.186) (end 137.165 85.857) (width 0.25) (layer "B.Cu") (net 27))
 (segment (start 137.165 85.857) (end 130.805 85.857) (width 0.25) (layer "B.Cu") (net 27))
 (segment (start 137.16 76.962) (end 142.494 76.962) (width 0.25) (layer "F.Cu") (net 28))
 (segment (start 130.805 83.317) (end 137.16 76.962) (width 0.25) (layer "F.Cu") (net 28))
 (segment (start 136.398 75.184) (end 142.494 75.184) (width 0.25) (layer "F.Cu") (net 29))
 (segment (start 130.805 80.777) (end 136.398 75.184) (width 0.25) (layer "F.Cu") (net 29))
 (segment (start 130.805 78.237) (end 135.636 73.406) (width 0.25) (layer "F.Cu") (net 30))
 (segment (start 135.636 73.406) (end 142.494 73.406) (width 0.25) (layer "F.Cu") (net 30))
 (segment (start 134.874 71.628) (end 142.494 71.628) (width 0.25) (layer "F.Cu") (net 31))
 (segment (start 130.805 75.697) (end 134.874 71.628) (width 0.25) (layer "F.Cu") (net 31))
 (segment (start 134.112 69.85) (end 142.494 69.85) (width 0.25) (layer "F.Cu") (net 32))
 (segment (start 130.805 73.157) (end 134.112 69.85) (width 0.25) (layer "F.Cu") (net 32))
 (segment (start 130.805 70.617) (end 133.35 68.072) (width 0.25) (layer "F.Cu") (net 33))
 (segment (start 133.35 68.072) (end 142.494 68.072) (width 0.25) (layer "F.Cu") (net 33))
 (segment (start 132.588 66.294) (end 142.494 66.294) (width 0.25) (layer "F.Cu") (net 34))
 (segment (start 130.805 68.077) (end 132.588 66.294) (width 0.25) (layer "F.Cu") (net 34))
 (segment (start 142.494 64.516) (end 133.096 64.516) (width 0.25) (layer "F.Cu") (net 35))
 (segment (start 133.096 64.516) (end 132.075 65.537) (width 0.25) (layer "F.Cu") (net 35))
 (segment (start 132.075 65.537) (end 130.805 65.537) (width 0.25) (layer "F.Cu") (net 35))
 (segment (start 123.444 105.41) (end 127.254 101.6) (width 0.25) (layer "B.Cu") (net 36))
 (segment (start 127.254 66.548) (end 130.805 62.997) (width 0.25) (layer "B.Cu") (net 36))
 (segment (start 127.254 101.6) (end 127.254 66.548) (width 0.25) (layer "B.Cu") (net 36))
 (segment (start 130.805 60.457) (end 137.663 60.457) (width 0.25) (layer "F.Cu") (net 37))
 (segment (start 137.663 60.457) (end 142.494 55.626) (width 0.25) (layer "F.Cu") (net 37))
 (segment (start 130.805 57.917) (end 141.981 57.917) (width 0.25) (layer "B.Cu") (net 38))
 (segment (start 141.981 57.917) (end 142.494 57.404) (width 0.25) (layer "B.Cu") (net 38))
 (segment (start 130.805 55.377) (end 129.680489 56.501511) (width 0.25) (layer "B.Cu") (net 39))
 (segment (start 129.680489 58.382789) (end 130.630189 59.332489) (width 0.25) (layer "B.Cu") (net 39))
 (segment (start 140.866489 59.332489) (end 142.494 60.96) (width 0.25) (layer "B.Cu") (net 39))
 (segment (start 130.630189 59.332489) (end 140.866489 59.332489) (width 0.25) (layer "B.Cu") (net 39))
 (segment (start 129.680489 56.501511) (end 129.680489 58.382789) (width 0.25) (layer "B.Cu") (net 39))
 (segment (start 123.444 87.63) (end 123.444 85.852) (width 0.25) (layer "B.Cu") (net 40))
 (segment (start 123.444 50.292) (end 128.26 50.292) (width 0.25) (layer "B.Cu") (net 40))
 (segment (start 123.444 85.852) (end 125.73 83.566) (width 0.25) (layer "B.Cu") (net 40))
 (segment (start 128.26 50.292) (end 130.805 52.837) (width 0.25) (layer "B.Cu") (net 40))
 (segment (start 125.73 83.566) (end 125.73 57.912) (width 0.25) (layer "B.Cu") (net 40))
 (segment (start 125.73 57.912) (end 130.805 52.837) (width 0.25) (layer "B.Cu") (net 40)))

